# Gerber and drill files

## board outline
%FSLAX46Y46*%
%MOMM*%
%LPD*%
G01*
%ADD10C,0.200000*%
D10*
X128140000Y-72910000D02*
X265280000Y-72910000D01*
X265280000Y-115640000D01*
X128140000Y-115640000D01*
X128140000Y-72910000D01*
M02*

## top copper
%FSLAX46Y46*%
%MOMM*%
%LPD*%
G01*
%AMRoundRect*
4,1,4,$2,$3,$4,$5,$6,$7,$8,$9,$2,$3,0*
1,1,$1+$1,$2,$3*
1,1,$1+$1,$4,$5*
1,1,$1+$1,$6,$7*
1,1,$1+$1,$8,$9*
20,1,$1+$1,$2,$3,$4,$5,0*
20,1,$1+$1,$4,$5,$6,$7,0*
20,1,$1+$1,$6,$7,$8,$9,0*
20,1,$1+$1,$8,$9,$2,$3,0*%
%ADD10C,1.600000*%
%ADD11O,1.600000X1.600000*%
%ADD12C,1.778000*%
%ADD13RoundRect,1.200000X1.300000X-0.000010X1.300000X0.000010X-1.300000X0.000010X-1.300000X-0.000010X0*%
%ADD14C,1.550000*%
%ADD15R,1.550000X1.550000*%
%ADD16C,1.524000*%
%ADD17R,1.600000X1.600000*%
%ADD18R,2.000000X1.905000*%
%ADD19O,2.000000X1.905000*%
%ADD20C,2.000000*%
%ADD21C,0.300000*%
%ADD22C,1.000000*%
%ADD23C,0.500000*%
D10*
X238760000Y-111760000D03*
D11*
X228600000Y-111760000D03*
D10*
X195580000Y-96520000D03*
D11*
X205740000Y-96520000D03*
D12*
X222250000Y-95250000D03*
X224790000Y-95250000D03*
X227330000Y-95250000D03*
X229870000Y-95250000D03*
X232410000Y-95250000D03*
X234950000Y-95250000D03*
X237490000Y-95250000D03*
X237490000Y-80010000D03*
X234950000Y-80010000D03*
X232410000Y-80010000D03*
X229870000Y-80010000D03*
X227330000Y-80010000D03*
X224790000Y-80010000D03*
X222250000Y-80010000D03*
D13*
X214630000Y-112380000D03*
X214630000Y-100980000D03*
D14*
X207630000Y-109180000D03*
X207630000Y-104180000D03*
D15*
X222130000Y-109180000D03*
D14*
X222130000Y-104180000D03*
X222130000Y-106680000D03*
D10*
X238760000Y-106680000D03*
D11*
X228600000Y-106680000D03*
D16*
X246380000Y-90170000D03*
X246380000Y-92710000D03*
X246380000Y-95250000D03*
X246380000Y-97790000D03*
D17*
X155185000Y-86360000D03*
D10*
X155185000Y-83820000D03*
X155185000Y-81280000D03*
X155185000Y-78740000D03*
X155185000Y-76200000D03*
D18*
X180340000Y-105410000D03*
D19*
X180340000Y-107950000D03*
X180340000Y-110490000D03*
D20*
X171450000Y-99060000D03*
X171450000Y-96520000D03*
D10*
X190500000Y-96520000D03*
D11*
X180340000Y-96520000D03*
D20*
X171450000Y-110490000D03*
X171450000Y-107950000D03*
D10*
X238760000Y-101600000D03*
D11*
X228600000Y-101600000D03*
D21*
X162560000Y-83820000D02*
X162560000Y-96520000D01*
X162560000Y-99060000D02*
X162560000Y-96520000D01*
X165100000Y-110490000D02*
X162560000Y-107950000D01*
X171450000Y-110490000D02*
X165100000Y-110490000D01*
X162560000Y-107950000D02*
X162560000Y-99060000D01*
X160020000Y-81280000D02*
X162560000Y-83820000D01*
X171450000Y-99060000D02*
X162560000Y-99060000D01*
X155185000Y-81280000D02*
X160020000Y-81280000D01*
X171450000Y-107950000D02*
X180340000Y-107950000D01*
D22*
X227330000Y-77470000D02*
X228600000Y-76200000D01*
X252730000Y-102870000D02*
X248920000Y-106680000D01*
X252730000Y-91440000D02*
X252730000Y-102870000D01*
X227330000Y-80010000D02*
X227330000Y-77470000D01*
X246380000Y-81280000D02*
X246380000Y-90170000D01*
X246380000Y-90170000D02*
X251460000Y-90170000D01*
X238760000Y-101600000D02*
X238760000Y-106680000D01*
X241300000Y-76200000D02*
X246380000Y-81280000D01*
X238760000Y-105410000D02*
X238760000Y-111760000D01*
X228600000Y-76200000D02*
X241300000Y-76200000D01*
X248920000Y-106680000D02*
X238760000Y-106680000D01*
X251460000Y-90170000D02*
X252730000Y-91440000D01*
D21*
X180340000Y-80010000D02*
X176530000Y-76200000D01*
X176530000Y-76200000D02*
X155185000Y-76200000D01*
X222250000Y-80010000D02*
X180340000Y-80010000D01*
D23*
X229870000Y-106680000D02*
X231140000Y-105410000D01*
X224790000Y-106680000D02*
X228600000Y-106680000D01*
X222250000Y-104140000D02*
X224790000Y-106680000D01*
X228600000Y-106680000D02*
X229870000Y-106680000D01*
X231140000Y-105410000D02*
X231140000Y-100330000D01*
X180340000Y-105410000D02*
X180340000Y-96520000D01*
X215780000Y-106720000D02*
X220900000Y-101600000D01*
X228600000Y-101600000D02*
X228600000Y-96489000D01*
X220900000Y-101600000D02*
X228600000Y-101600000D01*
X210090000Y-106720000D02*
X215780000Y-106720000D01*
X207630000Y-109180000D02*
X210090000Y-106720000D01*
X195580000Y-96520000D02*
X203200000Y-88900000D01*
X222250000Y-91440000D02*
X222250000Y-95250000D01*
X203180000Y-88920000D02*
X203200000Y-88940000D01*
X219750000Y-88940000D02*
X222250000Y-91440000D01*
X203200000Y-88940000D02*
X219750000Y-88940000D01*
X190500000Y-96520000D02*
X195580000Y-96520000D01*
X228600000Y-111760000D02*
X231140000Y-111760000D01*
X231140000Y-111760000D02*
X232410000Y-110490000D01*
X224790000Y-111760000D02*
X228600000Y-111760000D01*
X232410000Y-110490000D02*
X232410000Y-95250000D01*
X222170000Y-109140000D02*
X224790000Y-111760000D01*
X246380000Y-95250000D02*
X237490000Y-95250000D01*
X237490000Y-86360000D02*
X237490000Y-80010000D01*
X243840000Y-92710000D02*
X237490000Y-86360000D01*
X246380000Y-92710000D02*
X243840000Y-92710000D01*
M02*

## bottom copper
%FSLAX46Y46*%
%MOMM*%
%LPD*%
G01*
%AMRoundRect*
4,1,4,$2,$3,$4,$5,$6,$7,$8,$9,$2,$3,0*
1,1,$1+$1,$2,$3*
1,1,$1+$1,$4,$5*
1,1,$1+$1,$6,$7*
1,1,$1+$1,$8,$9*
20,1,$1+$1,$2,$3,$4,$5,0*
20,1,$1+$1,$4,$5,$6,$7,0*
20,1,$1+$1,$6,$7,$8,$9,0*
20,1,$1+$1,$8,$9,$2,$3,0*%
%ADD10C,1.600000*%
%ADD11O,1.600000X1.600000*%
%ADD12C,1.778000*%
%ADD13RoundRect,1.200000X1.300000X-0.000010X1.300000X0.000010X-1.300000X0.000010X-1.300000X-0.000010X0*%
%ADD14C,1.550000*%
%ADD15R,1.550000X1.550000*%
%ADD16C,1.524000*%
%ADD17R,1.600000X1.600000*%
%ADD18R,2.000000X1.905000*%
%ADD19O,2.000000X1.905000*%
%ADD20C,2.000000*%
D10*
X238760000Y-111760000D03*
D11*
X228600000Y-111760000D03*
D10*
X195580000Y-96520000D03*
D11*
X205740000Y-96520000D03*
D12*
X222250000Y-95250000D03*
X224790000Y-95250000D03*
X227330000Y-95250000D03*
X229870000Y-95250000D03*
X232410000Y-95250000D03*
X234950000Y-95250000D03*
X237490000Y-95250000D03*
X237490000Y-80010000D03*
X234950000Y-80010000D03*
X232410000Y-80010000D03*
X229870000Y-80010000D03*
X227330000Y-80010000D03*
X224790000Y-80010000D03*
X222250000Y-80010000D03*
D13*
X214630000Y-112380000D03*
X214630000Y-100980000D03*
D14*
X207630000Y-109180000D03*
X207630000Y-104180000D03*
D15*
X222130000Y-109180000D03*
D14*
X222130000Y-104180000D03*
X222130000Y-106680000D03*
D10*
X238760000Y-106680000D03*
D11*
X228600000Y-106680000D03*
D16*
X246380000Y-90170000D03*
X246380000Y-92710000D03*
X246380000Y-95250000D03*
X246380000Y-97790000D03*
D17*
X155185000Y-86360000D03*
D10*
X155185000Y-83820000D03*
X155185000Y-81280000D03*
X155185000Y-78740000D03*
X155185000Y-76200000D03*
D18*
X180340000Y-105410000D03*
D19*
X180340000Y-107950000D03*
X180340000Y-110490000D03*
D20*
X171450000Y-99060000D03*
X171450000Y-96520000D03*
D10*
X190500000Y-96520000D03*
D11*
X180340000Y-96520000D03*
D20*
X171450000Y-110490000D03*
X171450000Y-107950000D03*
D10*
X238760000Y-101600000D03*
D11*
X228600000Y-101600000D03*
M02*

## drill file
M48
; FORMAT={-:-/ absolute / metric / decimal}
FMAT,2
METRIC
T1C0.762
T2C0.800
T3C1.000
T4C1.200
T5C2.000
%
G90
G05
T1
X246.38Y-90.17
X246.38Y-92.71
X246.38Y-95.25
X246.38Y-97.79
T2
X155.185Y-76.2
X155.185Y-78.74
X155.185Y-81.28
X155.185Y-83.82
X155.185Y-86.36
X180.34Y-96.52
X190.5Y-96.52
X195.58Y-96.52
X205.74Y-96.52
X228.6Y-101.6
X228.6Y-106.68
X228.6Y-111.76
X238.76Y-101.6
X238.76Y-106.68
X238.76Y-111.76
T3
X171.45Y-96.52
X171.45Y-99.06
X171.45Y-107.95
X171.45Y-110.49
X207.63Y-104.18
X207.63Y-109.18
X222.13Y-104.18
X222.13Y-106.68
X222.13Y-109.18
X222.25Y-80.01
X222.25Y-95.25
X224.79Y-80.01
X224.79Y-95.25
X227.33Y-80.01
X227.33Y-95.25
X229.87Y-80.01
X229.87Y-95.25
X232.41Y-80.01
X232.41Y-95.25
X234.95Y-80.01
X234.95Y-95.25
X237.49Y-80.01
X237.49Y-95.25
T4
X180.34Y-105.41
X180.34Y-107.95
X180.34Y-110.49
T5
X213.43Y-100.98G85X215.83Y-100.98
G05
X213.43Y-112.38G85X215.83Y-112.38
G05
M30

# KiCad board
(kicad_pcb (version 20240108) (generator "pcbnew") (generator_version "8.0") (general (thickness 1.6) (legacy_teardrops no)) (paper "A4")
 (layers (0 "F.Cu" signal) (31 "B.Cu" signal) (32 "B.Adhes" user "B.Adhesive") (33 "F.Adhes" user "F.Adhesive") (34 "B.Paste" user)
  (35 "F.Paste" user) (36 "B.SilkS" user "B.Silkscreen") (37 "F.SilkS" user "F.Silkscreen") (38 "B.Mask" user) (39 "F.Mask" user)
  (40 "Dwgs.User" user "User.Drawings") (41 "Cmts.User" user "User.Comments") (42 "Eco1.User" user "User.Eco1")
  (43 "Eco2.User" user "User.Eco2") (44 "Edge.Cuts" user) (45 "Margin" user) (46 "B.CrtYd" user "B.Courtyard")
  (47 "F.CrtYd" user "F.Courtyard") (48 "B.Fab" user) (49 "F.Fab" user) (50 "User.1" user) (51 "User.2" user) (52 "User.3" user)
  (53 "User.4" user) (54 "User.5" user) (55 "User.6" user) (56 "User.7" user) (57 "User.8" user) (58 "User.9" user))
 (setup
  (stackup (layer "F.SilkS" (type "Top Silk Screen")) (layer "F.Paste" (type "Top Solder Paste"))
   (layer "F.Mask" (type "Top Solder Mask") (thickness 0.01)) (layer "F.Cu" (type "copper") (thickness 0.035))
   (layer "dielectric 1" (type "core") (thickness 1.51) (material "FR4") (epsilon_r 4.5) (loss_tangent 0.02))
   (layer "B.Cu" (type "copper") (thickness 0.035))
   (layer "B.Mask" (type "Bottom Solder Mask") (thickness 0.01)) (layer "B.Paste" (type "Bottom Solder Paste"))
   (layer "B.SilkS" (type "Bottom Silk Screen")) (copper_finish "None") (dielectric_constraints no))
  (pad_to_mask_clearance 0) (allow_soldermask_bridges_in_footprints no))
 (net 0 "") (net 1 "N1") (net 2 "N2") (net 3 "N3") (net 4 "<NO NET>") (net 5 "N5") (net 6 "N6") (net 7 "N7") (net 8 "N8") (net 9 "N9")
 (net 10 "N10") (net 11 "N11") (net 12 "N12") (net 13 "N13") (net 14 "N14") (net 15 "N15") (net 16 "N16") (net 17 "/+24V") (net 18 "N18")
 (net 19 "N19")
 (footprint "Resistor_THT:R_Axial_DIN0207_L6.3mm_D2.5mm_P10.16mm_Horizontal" (layer "F.Cu") (at 238.76 111.76 180)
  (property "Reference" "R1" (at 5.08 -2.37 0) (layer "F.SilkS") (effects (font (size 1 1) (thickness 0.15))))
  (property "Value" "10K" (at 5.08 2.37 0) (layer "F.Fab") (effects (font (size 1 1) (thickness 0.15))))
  (pad "1" thru_hole circle (at 0 0 180) (size 1.6 1.6) (drill 0.8) (layers "*.Cu" "*.Mask") (remove_unused_layers no) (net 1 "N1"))
  (pad "2" thru_hole oval (at 10.16 0 180) (size 1.6 1.6) (drill 0.8) (layers "*.Cu" "*.Mask") (remove_unused_layers no) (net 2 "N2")))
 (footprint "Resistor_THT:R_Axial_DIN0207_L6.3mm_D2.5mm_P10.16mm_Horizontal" (layer "F.Cu") (at 195.58 96.52)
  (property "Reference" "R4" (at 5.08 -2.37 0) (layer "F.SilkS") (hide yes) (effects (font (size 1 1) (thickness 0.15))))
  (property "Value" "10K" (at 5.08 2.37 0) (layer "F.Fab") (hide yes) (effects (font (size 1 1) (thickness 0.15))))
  (pad "1" thru_hole circle (at 0 0) (size 1.6 1.6) (drill 0.8) (layers "*.Cu" "*.Mask") (remove_unused_layers no) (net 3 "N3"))
  (pad "2" thru_hole oval (at 10.16 0) (size 1.6 1.6) (drill 0.8) (layers "*.Cu" "*.Mask") (remove_unused_layers no) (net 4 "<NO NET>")))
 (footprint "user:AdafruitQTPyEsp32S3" (layer "F.Cu") (at 222.25 95.25 90)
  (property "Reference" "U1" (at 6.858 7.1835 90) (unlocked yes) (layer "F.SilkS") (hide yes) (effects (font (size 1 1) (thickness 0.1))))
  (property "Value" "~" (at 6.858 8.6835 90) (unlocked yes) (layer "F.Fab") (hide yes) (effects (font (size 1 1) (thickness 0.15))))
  (pad "1" thru_hole circle (at 0 0 90) (size 1.778 1.778) (drill 1) (layers "*.Cu" "*.Mask") (remove_unused_layers no) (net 3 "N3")
   (solder_mask_margin 0.0508) (thermal_bridge_angle 0))
  (pad "2" thru_hole circle (at 0 2.54 90) (size 1.778 1.778) (drill 1) (layers "*.Cu" "*.Mask") (remove_unused_layers no) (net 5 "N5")
   (solder_mask_margin 0.0508) (thermal_bridge_angle 0))
  (pad "3" thru_hole circle (at 0 5.08 90) (size 1.778 1.778) (drill 1) (layers "*.Cu" "*.Mask") (remove_unused_layers no) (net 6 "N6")
   (solder_mask_margin 0.0508) (thermal_bridge_angle 0))
  (pad "4" thru_hole circle (at 0 7.62 90) (size 1.778 1.778) (drill 1) (layers "*.Cu" "*.Mask") (remove_unused_layers no) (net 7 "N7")
   (solder_mask_margin 0.0508) (thermal_bridge_angle 0))
  (pad "5" thru_hole circle (at 0 10.16 90) (size 1.778 1.778) (drill 1) (layers "*.Cu" "*.Mask") (remove_unused_layers no) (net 2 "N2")
   (solder_mask_margin 0.0508) (thermal_bridge_angle 0))
  (pad "6" thru_hole circle (at 0 12.7 90) (size 1.778 1.778) (drill 1) (layers "*.Cu" "*.Mask") (remove_unused_layers no) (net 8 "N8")
   (solder_mask_margin 0.0508) (thermal_bridge_angle 0))
  (pad "7" thru_hole circle (at 0 15.24 90) (size 1.778 1.778) (drill 1) (layers "*.Cu" "*.Mask") (remove_unused_layers no) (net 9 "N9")
   (solder_mask_margin 0.0508) (thermal_bridge_angle 0))
  (pad "8" thru_hole circle (at 15.24 15.24 270) (size 1.778 1.778) (drill 1) (layers "*.Cu" "*.Mask") (remove_unused_layers no)
   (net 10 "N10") (solder_mask_margin 0.0508) (thermal_bridge_angle 0))
  (pad "9" thru_hole circle (at 15.24 12.7 270) (size 1.778 1.778) (drill 1) (layers "*.Cu" "*.Mask") (remove_unused_layers no)
   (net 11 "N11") (solder_mask_margin 0.0508) (thermal_bridge_angle 0))
  (pad "10" thru_hole circle (at 15.24 10.16 270) (size 1.778 1.778) (drill 1) (layers "*.Cu" "*.Mask") (remove_unused_layers no)
   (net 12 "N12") (solder_mask_margin 0.0508) (thermal_bridge_angle 0))
  (pad "11" thru_hole circle (at 15.24 7.62 270) (size 1.778 1.778) (drill 1) (layers "*.Cu" "*.Mask") (remove_unused_layers no)
   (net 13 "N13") (solder_mask_margin 0.0508) (thermal_bridge_angle 0))
  (pad "12" thru_hole circle (at 15.24 5.08 270) (size 1.778 1.778) (drill 1) (layers "*.Cu" "*.Mask") (remove_unused_layers no)
   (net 1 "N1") (solder_mask_margin 0.0508) (thermal_bridge_angle 0))
  (pad "13" thru_hole circle (at 15.24 2.54 270) (size 1.778 1.778) (drill 1) (layers "*.Cu" "*.Mask") (remove_unused_layers no)
   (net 4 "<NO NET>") (solder_mask_margin 0.0508) (thermal_bridge_angle 0))
  (pad "14" thru_hole circle (at 15.24 0 270) (size 1.778 1.778) (drill 1) (layers "*.Cu" "*.Mask") (remove_unused_layers no) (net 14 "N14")
   (solder_mask_margin 0.0508) (thermal_bridge_angle 0)))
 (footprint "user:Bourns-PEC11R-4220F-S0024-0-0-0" (layer "F.Cu") (at 214.63 106.68 90)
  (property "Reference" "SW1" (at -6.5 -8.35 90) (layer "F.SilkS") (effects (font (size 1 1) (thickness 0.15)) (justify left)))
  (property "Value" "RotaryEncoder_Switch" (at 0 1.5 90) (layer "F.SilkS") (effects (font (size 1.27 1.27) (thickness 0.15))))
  (pad "" thru_hole roundrect (at -5.7 0 90) (size 2.4 5) (drill oval 2 4.4) (layers "*.Cu" "*.Mask") (remove_unused_layers no)
   (roundrect_rratio 0.5))
  (pad "" thru_hole roundrect (at 5.7 0 90) (size 2.4 5) (drill oval 2 4.4) (layers "*.Cu" "*.Mask") (remove_unused_layers no)
   (roundrect_rratio 0.5))
  (pad "1" thru_hole circle (at -2.5 -7 90) (size 1.55 1.55) (drill 1) (layers "*.Cu" "*.Mask") (remove_unused_layers no) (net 12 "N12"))
  (pad "2" thru_hole circle (at 2.5 -7 90) (size 1.55 1.55) (drill 1) (layers "*.Cu" "*.Mask") (remove_unused_layers no) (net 4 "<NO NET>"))
  (pad "A" thru_hole rect (at -2.5 7.5 90) (size 1.55 1.55) (drill 1) (layers "*.Cu" "*.Mask") (remove_unused_layers no) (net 2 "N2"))
  (pad "B" thru_hole circle (at 2.5 7.5 90) (size 1.55 1.55) (drill 1) (layers "*.Cu" "*.Mask") (remove_unused_layers no) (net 6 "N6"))
  (pad "C" thru_hole circle (at 0 7.5 90) (size 1.55 1.55) (drill 1) (layers "*.Cu" "*.Mask") (remove_unused_layers no) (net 4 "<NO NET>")))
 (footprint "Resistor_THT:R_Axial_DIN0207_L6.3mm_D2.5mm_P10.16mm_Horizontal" (layer "F.Cu") (at 238.76 106.68 180)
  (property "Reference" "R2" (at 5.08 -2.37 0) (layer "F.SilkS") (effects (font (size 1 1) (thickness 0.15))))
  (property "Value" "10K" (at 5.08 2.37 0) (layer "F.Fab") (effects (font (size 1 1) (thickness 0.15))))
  (pad "1" thru_hole circle (at 0 0 180) (size 1.6 1.6) (drill 0.8) (layers "*.Cu" "*.Mask") (remove_unused_layers no) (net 1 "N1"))
  (pad "2" thru_hole oval (at 10.16 0 180) (size 1.6 1.6) (drill 0.8) (layers "*.Cu" "*.Mask") (remove_unused_layers no) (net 6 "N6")))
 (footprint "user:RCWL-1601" (layer "F.Cu") (at 246.38 90.17 -90)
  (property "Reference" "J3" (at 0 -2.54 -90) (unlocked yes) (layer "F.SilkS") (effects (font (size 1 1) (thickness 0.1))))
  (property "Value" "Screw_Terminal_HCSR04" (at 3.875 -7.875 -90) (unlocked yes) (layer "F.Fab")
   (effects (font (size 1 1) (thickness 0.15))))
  (pad "1" thru_hole circle (at 0 0 270) (size 1.524 1.524) (drill 0.762) (layers "*.Cu" "*.Mask") (remove_unused_layers no) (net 1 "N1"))
  (pad "2" thru_hole circle (at 2.54 0 270) (size 1.524 1.524) (drill 0.762) (layers "*.Cu" "*.Mask") (remove_unused_layers no)
   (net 10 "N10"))
  (pad "3" thru_hole circle (at 5.08 0 270) (size 1.524 1.524) (drill 0.762) (layers "*.Cu" "*.Mask") (remove_unused_layers no) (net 9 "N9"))
  (pad "4" thru_hole circle (at 7.62 0 270) (size 1.524 1.524) (drill 0.762) (layers "*.Cu" "*.Mask") (remove_unused_layers no)
   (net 4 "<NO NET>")))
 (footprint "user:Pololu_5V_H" (layer "F.Cu") (at 155.185 81.28 90)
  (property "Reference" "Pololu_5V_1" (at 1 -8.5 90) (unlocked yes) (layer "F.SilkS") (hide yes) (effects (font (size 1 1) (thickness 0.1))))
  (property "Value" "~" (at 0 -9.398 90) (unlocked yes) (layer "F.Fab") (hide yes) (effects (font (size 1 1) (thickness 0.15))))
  (pad "1" thru_hole rect (at -5.08 0 90) (size 1.6 1.6) (drill 0.8) (layers "*.Cu" "*.Mask") (remove_unused_layers no) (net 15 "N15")
   (thermal_bridge_angle 45))
  (pad "2" thru_hole circle (at -2.54 0 90) (size 1.6 1.6) (drill 0.8) (layers "*.Cu" "*.Mask") (remove_unused_layers no) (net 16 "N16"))
  (pad "3" thru_hole circle (at 0 0 90) (size 1.6 1.6) (drill 0.8) (layers "*.Cu" "*.Mask") (remove_unused_layers no) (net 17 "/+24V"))
  (pad "4" thru_hole circle (at 2.54 0 90) (size 1.6 1.6) (drill 0.8) (layers "*.Cu" "*.Mask") (remove_unused_layers no) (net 4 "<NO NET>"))
  (pad "5" thru_hole circle (at 5.08 0 90) (size 1.6 1.6) (drill 0.8) (layers "*.Cu" "*.Mask") (remove_unused_layers no) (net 14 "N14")))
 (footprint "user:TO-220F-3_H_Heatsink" (layer "F.Cu") (at 180.34 105.41 -90)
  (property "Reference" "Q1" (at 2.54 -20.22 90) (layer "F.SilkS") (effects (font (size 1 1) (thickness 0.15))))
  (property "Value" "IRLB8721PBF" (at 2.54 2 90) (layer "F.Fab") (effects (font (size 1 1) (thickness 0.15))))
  (pad "1" thru_hole rect (at 0 0 270) (size 1.905 2) (drill 1.2) (layers "*.Cu" "*.Mask") (remove_unused_layers no) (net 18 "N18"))
  (pad "2" thru_hole oval (at 2.54 0 270) (size 1.905 2) (drill 1.2) (layers "*.Cu" "*.Mask") (remove_unused_layers no) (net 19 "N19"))
  (pad "3" thru_hole oval (at 5.08 0 270) (size 1.905 2) (drill 1.2) (layers "*.Cu" "*.Mask") (remove_unused_layers no) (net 4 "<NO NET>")))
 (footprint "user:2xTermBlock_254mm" (layer "F.Cu") (at 171.45 99.06 90)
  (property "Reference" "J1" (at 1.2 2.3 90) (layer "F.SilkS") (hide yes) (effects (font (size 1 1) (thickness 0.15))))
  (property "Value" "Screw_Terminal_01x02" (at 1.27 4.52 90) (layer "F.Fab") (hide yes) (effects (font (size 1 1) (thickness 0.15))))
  (pad "1" thru_hole circle (at 0 0 90) (size 2 2) (drill 1) (layers "*.Cu" "*.Mask") (remove_unused_layers no) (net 17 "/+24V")
   (thermal_bridge_angle 90))
  (pad "2" thru_hole circle (at 2.54 0 90) (size 2 2) (drill 1) (layers "*.Cu" "*.Mask") (remove_unused_layers no) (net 4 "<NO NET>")))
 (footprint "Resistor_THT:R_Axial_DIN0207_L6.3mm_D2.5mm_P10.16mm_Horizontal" (layer "F.Cu") (at 190.5 96.52 180)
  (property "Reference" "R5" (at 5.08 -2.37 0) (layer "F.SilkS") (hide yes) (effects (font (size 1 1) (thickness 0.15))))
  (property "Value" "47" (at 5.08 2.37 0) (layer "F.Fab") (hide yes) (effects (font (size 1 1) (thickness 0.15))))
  (pad "1" thru_hole circle (at 0 0 180) (size 1.6 1.6) (drill 0.8) (layers "*.Cu" "*.Mask") (remove_unused_layers no) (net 3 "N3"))
  (pad "2" thru_hole oval (at 10.16 0 180) (size 1.6 1.6) (drill 0.8) (layers "*.Cu" "*.Mask") (remove_unused_layers no) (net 18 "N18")))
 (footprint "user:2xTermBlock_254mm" (layer "F.Cu") (at 171.45 110.49 90)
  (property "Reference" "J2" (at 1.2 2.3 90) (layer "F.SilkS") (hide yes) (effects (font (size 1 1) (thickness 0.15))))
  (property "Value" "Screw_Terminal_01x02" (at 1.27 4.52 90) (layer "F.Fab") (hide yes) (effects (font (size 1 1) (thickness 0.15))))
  (pad "1" thru_hole circle (at 0 0 90) (size 2 2) (drill 1) (layers "*.Cu" "*.Mask") (remove_unused_layers no) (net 17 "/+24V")
   (thermal_bridge_angle 90))
  (pad "2" thru_hole circle (at 2.54 0 90) (size 2 2) (drill 1) (layers "*.Cu" "*.Mask") (remove_unused_layers no) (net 19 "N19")))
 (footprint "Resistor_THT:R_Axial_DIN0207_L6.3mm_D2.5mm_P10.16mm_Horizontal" (layer "F.Cu") (at 238.76 101.6 180)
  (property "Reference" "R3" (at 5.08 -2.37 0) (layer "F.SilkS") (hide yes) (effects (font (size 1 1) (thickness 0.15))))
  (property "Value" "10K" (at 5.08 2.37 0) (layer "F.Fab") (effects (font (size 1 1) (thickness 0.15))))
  (pad "1" thru_hole circle (at 0 0 180) (size 1.6 1.6) (drill 0.8) (layers "*.Cu" "*.Mask") (remove_unused_layers no) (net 1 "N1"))
  (pad "2" thru_hole oval (at 10.16 0 180) (size 1.6 1.6) (drill 0.8) (layers "*.Cu" "*.Mask") (remove_unused_layers no) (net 12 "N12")))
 (gr_rect (start 128.14 72.91) (end 265.28 115.64) (stroke (width 0.2) (type default)) (fill none) (layer "Edge.Cuts"))
 (segment (start 162.56 83.82) (end 162.56 96.52) (width 0.3) (layer "F.Cu") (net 17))
 (segment (start 162.56 99.06) (end 162.56 96.52) (width 0.3) (layer "F.Cu") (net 17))
 (segment (start 165.1 110.49) (end 162.56 107.95) (width 0.3) (layer "F.Cu") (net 17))
 (segment (start 171.45 110.49) (end 165.1 110.49) (width 0.3) (layer "F.Cu") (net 17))
 (segment (start 162.56 107.95) (end 162.56 99.06) (width 0.3) (layer "F.Cu") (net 17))
 (segment (start 160.02 81.28) (end 162.56 83.82) (width 0.3) (layer "F.Cu") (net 17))
 (segment (start 171.45 99.06) (end 162.56 99.06) (width 0.3) (layer "F.Cu") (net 17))
 (segment (start 155.185 81.28) (end 160.02 81.28) (width 0.3) (layer "F.Cu") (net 17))
 (segment (start 171.45 107.95) (end 180.34 107.95) (width 0.3) (layer "F.Cu") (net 19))
 (segment (start 227.33 77.47) (end 228.6 76.2) (width 1) (layer "F.Cu") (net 1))
 (segment (start 252.73 102.87) (end 248.92 106.68) (width 1) (layer "F.Cu") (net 1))
 (segment (start 252.73 91.44) (end 252.73 102.87) (width 1) (layer "F.Cu") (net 1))
 (segment (start 227.33 80.01) (end 227.33 77.47) (width 1) (layer "F.Cu") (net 1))
 (segment (start 246.38 81.28) (end 246.38 90.17) (width 1) (layer "F.Cu") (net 1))
 (segment (start 246.38 90.17) (end 251.46 90.17) (width 1) (layer "F.Cu") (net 1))
 (segment (start 238.76 101.6) (end 238.76 106.68) (width 1) (layer "F.Cu") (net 1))
 (segment (start 241.3 76.2) (end 246.38 81.28) (width 1) (layer "F.Cu") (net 1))
 (segment (start 238.76 105.41) (end 238.76 111.76) (width 1) (layer "F.Cu") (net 1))
 (segment (start 228.6 76.2) (end 241.3 76.2) (width 1) (layer "F.Cu") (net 1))
 (segment (start 248.92 106.68) (end 238.76 106.68) (width 1) (layer "F.Cu") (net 1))
 (segment (start 251.46 90.17) (end 252.73 91.44) (width 1) (layer "F.Cu") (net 1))
 (segment (start 180.34 80.01) (end 176.53 76.2) (width 0.3) (layer "F.Cu") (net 14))
 (segment (start 176.53 76.2) (end 155.185 76.2) (width 0.3) (layer "F.Cu") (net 14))
 (segment (start 222.25 80.01) (end 180.34 80.01) (width 0.3) (layer "F.Cu") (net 14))
 (segment (start 229.87 106.68) (end 231.14 105.41) (width 0.5) (layer "F.Cu") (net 6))
 (segment (start 224.79 106.68) (end 228.6 106.68) (width 0.5) (layer "F.Cu") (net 6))
 (segment (start 222.25 104.14) (end 224.79 106.68) (width 0.5) (layer "F.Cu") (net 6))
 (segment (start 228.6 106.68) (end 229.87 106.68) (width 0.5) (layer "F.Cu") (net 6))
 (segment (start 231.14 105.41) (end 231.14 100.33) (width 0.5) (layer "F.Cu") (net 6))
 (segment (start 180.34 105.41) (end 180.34 96.52) (width 0.5) (layer "F.Cu") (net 18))
 (segment (start 215.78 106.72) (end 220.9 101.6) (width 0.5) (layer "F.Cu") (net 12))
 (segment (start 228.6 101.6) (end 228.6 96.489) (width 0.5) (layer "F.Cu") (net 12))
 (segment (start 220.9 101.6) (end 228.6 101.6) (width 0.5) (layer "F.Cu") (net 12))
 (segment (start 210.09 106.72) (end 215.78 106.72) (width 0.5) (layer "F.Cu") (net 12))
 (segment (start 207.63 109.18) (end 210.09 106.72) (width 0.5) (layer "F.Cu") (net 12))
 (segment (start 195.58 96.52) (end 203.2 88.9) (width 0.5) (layer "F.Cu") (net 3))
 (segment (start 222.25 91.44) (end 222.25 95.25) (width 0.5) (layer "F.Cu") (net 3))
 (segment (start 203.18 88.92) (end 203.2 88.94) (width 0.5) (layer "F.Cu") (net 3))
 (segment (start 219.75 88.94) (end 222.25 91.44) (width 0.5) (layer "F.Cu") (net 3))
 (segment (start 203.2 88.94) (end 219.75 88.94) (width 0.5) (layer "F.Cu") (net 3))
 (segment (start 190.5 96.52) (end 195.58 96.52) (width 0.5) (layer "F.Cu") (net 3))
 (segment (start 228.6 111.76) (end 231.14 111.76) (width 0.5) (layer "F.Cu") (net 2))
 (segment (start 231.14 111.76) (end 232.41 110.49) (width 0.5) (layer "F.Cu") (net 2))
 (segment (start 224.79 111.76) (end 228.6 111.76) (width 0.5) (layer "F.Cu") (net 2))
 (segment (start 232.41 110.49) (end 232.41 95.25) (width 0.5) (layer "F.Cu") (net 2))
 (segment (start 222.17 109.14) (end 224.79 111.76) (width 0.5) (layer "F.Cu") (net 2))
 (segment (start 246.38 95.25) (end 237.49 95.25) (width 0.5) (layer "F.Cu") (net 9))
 (segment (start 237.49 86.36) (end 237.49 80.01) (width 0.5) (layer "F.Cu") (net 10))
 (segment (start 243.84 92.71) (end 237.49 86.36) (width 0.5) (layer "F.Cu") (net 10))
 (segment (start 246.38 92.71) (end 243.84 92.71) (width 0.5) (layer "F.Cu") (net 10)))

